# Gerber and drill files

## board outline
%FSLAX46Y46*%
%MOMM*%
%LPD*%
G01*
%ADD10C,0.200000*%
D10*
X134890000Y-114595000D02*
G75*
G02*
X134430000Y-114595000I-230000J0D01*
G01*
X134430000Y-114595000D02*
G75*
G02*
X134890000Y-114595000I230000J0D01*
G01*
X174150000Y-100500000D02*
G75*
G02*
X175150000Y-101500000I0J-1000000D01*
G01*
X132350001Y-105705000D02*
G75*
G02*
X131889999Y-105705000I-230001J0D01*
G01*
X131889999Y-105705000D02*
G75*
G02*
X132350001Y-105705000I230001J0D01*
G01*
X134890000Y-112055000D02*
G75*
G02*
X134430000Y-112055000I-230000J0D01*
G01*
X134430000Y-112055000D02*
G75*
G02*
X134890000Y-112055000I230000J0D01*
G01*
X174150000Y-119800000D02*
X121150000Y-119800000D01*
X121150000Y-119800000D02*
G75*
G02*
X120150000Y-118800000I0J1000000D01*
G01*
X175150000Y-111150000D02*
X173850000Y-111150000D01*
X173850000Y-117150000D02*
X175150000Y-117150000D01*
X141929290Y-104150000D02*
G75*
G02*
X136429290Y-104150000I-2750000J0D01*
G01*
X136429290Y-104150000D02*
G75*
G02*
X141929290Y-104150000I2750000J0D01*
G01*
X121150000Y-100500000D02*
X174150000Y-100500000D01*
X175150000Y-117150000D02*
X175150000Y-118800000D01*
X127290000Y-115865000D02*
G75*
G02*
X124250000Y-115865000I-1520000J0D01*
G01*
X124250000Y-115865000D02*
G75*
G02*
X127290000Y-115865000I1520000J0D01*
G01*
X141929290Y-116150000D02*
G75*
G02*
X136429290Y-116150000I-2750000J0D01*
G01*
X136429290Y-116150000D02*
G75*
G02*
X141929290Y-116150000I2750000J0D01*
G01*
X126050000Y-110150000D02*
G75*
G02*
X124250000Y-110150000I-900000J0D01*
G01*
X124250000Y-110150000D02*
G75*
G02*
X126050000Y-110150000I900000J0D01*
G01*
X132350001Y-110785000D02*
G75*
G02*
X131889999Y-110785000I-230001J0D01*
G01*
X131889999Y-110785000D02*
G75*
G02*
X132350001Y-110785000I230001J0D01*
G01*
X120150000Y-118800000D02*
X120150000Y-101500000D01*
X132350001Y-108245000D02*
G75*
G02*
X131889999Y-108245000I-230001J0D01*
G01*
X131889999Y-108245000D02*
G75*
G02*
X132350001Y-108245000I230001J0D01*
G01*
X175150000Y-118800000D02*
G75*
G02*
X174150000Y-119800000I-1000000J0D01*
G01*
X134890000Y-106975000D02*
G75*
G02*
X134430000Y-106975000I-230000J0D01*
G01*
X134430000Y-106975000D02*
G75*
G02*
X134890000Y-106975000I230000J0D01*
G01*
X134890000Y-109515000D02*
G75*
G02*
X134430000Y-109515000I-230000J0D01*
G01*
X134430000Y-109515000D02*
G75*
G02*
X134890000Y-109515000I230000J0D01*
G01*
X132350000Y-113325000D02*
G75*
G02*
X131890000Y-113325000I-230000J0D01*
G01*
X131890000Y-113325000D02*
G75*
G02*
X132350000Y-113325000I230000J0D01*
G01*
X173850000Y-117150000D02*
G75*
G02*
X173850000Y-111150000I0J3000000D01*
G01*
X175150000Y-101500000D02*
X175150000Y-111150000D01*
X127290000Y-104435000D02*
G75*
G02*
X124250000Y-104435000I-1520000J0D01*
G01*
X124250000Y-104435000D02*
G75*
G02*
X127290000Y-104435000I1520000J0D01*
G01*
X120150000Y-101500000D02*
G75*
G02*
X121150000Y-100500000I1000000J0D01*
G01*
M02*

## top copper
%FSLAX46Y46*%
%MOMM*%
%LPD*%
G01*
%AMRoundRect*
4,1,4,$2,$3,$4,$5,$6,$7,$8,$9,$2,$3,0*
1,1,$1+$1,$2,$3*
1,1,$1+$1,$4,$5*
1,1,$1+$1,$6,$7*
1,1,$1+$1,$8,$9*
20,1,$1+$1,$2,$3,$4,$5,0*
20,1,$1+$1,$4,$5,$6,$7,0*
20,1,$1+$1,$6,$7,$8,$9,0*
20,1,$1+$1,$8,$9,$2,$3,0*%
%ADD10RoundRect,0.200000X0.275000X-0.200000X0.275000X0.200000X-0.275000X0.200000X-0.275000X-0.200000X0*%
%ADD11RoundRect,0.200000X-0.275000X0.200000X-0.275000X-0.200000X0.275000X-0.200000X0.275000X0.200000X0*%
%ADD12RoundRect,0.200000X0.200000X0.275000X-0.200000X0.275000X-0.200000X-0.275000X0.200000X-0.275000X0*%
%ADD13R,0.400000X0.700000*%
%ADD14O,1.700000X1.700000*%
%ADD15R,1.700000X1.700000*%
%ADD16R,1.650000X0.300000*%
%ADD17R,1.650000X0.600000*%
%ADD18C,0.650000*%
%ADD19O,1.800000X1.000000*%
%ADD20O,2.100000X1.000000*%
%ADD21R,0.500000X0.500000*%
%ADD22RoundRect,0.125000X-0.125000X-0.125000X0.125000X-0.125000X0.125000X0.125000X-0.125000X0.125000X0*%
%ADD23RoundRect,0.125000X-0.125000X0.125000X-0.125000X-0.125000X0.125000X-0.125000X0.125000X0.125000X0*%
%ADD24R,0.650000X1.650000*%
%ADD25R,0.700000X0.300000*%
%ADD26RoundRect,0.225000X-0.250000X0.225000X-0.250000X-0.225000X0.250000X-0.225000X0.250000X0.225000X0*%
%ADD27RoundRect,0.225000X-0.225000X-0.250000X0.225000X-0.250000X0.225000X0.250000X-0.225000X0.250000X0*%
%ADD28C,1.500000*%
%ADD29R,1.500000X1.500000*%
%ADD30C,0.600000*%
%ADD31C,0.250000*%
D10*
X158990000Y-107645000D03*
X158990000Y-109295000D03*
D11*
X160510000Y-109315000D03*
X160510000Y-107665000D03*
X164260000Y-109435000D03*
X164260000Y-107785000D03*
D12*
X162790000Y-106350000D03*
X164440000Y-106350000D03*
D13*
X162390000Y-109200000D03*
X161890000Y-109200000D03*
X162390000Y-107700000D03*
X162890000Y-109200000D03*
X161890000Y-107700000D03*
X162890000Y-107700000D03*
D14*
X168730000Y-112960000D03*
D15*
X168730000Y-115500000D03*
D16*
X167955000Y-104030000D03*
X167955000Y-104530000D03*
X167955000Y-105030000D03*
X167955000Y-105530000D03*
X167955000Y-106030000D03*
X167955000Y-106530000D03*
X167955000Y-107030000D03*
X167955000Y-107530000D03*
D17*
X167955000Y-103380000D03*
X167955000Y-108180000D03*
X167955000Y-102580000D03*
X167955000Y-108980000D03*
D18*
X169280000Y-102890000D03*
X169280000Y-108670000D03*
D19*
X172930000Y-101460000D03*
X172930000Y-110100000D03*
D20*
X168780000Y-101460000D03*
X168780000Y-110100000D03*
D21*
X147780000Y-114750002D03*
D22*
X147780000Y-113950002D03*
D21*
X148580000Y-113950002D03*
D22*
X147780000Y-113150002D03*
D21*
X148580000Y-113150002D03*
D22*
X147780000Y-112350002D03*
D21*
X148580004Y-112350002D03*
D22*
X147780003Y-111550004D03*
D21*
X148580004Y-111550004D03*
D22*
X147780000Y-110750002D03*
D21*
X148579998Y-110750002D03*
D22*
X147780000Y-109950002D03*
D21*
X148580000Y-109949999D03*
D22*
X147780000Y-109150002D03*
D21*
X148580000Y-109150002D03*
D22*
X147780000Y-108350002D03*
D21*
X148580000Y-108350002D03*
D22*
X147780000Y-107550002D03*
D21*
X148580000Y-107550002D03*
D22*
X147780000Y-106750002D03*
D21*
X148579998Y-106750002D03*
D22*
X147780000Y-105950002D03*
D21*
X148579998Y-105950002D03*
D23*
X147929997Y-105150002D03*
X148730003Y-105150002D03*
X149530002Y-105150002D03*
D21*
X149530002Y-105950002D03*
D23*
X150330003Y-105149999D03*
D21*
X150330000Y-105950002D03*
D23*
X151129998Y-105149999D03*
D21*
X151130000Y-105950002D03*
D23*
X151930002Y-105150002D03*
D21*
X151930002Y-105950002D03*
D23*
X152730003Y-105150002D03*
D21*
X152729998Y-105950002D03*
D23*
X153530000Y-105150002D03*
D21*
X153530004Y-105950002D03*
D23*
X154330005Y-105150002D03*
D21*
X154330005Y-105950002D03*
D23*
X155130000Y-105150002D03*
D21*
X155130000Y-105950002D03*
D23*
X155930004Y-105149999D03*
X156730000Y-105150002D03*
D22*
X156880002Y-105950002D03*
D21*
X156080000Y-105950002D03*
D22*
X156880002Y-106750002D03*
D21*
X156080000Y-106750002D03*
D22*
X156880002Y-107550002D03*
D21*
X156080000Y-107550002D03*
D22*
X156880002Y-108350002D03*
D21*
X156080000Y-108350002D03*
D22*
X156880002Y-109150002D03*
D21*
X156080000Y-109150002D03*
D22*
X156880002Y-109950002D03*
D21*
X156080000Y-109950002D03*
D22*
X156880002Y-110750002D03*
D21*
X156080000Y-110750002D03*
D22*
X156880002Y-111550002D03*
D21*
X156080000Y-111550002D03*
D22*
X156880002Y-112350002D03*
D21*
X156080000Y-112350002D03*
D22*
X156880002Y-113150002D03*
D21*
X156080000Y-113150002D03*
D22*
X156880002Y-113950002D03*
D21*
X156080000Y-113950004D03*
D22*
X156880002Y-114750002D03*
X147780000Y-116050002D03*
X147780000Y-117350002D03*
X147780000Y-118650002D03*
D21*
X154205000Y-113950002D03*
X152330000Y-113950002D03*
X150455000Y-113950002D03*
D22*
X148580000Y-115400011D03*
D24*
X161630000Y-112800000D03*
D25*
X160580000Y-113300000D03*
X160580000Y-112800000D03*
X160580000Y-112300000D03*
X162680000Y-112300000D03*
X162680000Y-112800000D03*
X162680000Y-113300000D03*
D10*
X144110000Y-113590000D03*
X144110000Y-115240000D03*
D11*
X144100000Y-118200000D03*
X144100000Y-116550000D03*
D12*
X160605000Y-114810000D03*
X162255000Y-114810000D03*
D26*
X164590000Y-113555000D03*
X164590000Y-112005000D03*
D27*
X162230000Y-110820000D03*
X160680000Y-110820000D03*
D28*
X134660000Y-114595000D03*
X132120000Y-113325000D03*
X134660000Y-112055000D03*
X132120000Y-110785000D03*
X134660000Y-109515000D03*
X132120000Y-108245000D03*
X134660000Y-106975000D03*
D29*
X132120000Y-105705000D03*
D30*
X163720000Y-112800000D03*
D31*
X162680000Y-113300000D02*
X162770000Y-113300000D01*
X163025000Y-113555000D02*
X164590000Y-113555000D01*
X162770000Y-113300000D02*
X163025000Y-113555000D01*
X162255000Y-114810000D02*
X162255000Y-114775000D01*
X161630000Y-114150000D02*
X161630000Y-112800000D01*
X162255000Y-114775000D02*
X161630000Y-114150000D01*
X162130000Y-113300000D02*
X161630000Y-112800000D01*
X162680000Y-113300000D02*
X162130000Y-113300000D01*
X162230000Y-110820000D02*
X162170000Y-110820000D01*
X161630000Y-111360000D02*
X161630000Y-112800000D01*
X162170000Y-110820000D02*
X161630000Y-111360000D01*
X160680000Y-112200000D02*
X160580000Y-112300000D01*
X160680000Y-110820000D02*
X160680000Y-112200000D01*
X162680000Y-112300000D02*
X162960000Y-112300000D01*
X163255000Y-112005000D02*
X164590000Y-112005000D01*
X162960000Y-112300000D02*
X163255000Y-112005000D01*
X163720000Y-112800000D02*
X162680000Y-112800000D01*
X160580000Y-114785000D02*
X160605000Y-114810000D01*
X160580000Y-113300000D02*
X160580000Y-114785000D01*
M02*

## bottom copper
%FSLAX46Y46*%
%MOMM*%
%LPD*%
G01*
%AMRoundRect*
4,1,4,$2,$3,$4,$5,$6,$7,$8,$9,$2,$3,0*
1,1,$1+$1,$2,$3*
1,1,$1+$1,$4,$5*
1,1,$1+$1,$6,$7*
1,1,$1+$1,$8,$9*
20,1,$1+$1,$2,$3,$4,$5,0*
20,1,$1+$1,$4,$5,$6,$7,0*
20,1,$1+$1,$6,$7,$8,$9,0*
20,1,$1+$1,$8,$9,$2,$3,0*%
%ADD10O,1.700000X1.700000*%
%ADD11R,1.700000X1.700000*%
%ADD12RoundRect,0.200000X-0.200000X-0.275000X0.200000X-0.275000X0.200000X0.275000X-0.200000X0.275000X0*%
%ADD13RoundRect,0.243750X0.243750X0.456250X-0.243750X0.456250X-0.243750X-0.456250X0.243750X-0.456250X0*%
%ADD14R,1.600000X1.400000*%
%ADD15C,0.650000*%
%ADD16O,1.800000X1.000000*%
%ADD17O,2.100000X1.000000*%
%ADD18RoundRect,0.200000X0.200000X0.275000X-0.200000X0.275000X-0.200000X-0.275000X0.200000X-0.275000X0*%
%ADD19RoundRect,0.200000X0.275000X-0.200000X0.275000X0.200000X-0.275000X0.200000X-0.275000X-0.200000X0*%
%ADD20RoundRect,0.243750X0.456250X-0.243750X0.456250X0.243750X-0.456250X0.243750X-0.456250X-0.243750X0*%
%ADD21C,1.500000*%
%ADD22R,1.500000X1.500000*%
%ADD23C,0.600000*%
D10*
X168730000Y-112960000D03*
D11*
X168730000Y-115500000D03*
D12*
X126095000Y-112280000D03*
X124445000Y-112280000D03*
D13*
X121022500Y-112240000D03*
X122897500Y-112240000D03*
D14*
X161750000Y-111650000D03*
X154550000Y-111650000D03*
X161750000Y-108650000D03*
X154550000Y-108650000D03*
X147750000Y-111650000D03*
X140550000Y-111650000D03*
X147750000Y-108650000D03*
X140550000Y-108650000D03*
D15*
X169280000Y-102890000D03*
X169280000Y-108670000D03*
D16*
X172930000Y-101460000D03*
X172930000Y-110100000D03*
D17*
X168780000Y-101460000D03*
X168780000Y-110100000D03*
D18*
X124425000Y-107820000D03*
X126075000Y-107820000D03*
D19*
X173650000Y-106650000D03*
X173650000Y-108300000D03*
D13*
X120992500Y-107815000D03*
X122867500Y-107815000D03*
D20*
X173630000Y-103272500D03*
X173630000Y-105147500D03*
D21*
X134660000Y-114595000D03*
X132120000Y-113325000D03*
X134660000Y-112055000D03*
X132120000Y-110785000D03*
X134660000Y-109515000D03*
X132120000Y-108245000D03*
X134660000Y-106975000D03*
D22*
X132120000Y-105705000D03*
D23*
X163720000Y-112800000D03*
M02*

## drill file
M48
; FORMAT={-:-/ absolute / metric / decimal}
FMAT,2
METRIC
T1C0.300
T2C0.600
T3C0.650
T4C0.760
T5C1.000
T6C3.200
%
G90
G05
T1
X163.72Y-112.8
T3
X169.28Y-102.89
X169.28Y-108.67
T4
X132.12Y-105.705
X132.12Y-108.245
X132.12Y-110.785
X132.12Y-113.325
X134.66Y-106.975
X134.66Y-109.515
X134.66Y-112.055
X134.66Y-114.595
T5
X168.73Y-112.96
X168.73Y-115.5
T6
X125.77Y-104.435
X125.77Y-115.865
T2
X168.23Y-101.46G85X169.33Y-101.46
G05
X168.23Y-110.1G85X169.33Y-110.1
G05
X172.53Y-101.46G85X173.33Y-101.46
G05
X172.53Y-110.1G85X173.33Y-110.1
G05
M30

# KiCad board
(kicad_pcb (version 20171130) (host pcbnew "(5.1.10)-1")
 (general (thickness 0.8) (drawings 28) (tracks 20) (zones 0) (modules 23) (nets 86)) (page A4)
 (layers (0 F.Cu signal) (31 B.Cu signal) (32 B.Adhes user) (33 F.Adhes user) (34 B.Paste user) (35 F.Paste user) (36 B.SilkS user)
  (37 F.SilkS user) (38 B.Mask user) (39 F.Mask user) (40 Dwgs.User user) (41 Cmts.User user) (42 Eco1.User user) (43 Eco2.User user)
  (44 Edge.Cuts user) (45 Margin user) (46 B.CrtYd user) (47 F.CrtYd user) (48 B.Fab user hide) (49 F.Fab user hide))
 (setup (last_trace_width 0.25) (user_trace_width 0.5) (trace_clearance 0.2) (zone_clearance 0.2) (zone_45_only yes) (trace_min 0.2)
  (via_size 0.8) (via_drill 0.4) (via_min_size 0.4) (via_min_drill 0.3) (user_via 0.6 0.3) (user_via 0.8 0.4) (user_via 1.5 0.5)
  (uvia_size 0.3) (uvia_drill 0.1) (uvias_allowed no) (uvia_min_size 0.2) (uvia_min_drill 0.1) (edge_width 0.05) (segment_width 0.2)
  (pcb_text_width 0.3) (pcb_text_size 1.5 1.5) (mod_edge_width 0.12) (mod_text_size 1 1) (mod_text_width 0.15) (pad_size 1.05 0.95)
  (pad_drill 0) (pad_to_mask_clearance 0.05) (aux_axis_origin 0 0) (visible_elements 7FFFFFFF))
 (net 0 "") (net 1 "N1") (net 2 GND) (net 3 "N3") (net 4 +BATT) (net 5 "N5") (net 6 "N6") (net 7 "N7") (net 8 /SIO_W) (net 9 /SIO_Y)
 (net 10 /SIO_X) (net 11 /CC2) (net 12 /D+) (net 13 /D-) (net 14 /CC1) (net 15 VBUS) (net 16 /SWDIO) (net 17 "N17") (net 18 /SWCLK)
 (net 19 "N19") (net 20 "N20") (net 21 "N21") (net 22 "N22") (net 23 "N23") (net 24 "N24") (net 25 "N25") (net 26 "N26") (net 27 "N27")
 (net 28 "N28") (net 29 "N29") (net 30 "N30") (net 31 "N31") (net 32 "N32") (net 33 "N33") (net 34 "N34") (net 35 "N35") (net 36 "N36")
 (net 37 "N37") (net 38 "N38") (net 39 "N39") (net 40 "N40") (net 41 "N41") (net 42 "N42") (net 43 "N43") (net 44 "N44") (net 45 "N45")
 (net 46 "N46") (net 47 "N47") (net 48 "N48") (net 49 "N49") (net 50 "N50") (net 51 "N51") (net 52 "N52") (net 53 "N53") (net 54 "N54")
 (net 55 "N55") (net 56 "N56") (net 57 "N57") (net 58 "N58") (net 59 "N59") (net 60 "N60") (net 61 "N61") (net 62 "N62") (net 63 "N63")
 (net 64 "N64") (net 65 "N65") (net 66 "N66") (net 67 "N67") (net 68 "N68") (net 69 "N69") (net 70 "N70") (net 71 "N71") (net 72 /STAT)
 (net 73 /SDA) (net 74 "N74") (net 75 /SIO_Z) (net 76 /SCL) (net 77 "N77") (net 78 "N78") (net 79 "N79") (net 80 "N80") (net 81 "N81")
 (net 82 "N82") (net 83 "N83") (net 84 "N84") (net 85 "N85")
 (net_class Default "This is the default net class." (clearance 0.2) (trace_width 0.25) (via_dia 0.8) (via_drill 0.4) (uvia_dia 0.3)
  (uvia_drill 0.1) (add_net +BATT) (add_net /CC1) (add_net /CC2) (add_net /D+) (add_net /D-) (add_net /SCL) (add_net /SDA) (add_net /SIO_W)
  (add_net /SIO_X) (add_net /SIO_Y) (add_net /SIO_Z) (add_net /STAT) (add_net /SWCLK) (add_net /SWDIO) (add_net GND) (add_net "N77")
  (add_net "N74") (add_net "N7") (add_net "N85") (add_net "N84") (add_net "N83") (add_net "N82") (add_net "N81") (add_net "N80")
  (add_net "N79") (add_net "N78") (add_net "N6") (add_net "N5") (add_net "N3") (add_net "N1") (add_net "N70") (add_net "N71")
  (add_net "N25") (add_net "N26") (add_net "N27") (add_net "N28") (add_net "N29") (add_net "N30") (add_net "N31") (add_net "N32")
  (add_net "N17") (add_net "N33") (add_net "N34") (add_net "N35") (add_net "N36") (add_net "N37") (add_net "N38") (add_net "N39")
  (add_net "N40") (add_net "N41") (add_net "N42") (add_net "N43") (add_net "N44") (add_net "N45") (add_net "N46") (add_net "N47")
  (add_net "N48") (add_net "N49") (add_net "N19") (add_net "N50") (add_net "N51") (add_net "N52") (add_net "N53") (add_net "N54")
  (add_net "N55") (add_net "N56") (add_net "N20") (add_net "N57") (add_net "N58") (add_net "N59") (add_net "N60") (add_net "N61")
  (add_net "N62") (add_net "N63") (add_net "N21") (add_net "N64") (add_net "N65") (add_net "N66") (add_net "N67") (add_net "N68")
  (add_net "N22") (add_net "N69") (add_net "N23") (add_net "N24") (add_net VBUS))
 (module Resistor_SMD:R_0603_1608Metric (layer F.Cu) (at 158.99 108.47 90)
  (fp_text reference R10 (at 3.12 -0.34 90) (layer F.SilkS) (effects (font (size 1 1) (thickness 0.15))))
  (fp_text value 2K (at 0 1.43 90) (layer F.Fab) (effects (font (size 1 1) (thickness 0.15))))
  (pad 2 smd roundrect (at 0.825 0 90) (size 0.8 0.95) (layers F.Cu F.Paste F.Mask) (roundrect_rratio 0.25) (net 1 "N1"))
  (pad 1 smd roundrect (at -0.825 0 90) (size 0.8 0.95) (layers F.Cu F.Paste F.Mask) (roundrect_rratio 0.25) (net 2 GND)))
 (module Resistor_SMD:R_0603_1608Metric (layer F.Cu) (at 160.51 108.49 270)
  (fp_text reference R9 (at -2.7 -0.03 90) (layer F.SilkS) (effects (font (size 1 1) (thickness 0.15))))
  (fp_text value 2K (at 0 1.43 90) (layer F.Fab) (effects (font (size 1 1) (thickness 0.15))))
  (pad 2 smd roundrect (at 0.825 0 270) (size 0.8 0.95) (layers F.Cu F.Paste F.Mask) (roundrect_rratio 0.25) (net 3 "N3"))
  (pad 1 smd roundrect (at -0.825 0 270) (size 0.8 0.95) (layers F.Cu F.Paste F.Mask) (roundrect_rratio 0.25) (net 1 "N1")))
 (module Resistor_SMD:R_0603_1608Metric (layer F.Cu) (at 164.26 108.61 270)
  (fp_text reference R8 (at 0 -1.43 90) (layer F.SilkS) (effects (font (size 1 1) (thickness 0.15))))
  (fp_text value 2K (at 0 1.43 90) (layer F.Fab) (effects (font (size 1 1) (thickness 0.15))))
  (pad 2 smd roundrect (at 0.825 0 270) (size 0.8 0.95) (layers F.Cu F.Paste F.Mask) (roundrect_rratio 0.25) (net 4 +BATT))
  (pad 1 smd roundrect (at -0.825 0 270) (size 0.8 0.95) (layers F.Cu F.Paste F.Mask) (roundrect_rratio 0.25) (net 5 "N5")))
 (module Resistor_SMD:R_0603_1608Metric (layer F.Cu) (at 163.615 106.35 180)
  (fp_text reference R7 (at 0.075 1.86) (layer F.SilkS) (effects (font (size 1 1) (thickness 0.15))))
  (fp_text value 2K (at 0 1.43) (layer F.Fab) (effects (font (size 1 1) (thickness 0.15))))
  (pad 2 smd roundrect (at 0.825 0 180) (size 0.8 0.95) (layers F.Cu F.Paste F.Mask) (roundrect_rratio 0.25) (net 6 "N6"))
  (pad 1 smd roundrect (at -0.825 0 180) (size 0.8 0.95) (layers F.Cu F.Paste F.Mask) (roundrect_rratio 0.25) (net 2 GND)))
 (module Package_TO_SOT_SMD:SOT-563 (layer F.Cu) (at 162.39 108.45 270)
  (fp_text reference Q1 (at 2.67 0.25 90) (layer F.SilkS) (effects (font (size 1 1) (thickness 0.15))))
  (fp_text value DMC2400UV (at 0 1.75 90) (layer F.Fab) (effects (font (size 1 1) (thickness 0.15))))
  (pad 5 smd rect (at 0.75 0 270) (size 0.7 0.4) (layers F.Cu F.Paste F.Mask) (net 5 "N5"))
  (pad 4 smd rect (at 0.75 0.5 270) (size 0.7 0.4) (layers F.Cu F.Paste F.Mask) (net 3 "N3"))
  (pad 2 smd rect (at -0.75 0 270) (size 0.7 0.4) (layers F.Cu F.Paste F.Mask) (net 6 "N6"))
  (pad 6 smd rect (at 0.75 -0.5 270) (size 0.7 0.4) (layers F.Cu F.Paste F.Mask) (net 4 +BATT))
  (pad 3 smd rect (at -0.75 0.5 270) (size 0.7 0.4) (layers F.Cu F.Paste F.Mask) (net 5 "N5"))
  (pad 1 smd rect (at -0.75 -0.5 270) (size 0.7 0.4) (layers F.Cu F.Paste F.Mask) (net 2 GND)))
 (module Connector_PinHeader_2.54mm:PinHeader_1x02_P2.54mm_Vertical (layer F.Cu) (at 168.73 115.5 180)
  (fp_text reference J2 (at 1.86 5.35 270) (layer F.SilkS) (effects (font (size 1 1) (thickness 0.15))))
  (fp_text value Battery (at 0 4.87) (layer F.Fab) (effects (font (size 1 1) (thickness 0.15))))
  (pad 2 thru_hole oval (at 0 2.54 180) (size 1.7 1.7) (drill 1) (layers *.Cu *.Mask) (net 4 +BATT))
  (pad 1 thru_hole rect (at 0 0 180) (size 1.7 1.7) (drill 1) (layers *.Cu *.Mask) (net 2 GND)))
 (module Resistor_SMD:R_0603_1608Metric (layer B.Cu) (at 125.27 112.28)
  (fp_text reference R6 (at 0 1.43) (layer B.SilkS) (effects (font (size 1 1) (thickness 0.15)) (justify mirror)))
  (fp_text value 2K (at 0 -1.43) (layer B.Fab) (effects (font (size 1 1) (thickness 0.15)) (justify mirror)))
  (pad 2 smd roundrect (at 0.825 0) (size 0.8 0.95) (layers B.Cu B.Paste B.Mask) (roundrect_rratio 0.25) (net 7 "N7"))
  (pad 1 smd roundrect (at -0.825 0) (size 0.8 0.95) (layers B.Cu B.Paste B.Mask) (roundrect_rratio 0.25) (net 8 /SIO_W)))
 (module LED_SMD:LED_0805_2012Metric (layer B.Cu) (at 121.96 112.24 180)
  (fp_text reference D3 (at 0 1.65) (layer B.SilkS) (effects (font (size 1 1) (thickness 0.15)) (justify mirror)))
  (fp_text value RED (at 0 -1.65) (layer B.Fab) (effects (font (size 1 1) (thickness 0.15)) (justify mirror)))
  (pad 2 smd roundrect (at 0.9375 0 180) (size 0.975 1.4) (layers B.Cu B.Paste B.Mask) (roundrect_rratio 0.25) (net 4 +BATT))
  (pad 1 smd roundrect (at -0.9375 0 180) (size 0.975 1.4) (layers B.Cu B.Paste B.Mask) (roundrect_rratio 0.25) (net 7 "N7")))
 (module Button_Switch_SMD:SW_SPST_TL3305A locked (layer B.Cu) (at 158.15 110.15 180)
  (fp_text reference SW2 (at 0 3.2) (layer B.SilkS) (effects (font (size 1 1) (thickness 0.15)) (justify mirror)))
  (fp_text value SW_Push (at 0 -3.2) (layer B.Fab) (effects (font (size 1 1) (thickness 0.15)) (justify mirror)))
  (pad 2 smd rect (at -3.6 -1.5 180) (size 1.6 1.4) (layers B.Cu B.Paste B.Mask) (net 2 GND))
  (pad 2 smd rect (at 3.6 -1.5 180) (size 1.6 1.4) (layers B.Cu B.Paste B.Mask) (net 2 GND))
  (pad 1 smd rect (at -3.6 1.5 180) (size 1.6 1.4) (layers B.Cu B.Paste B.Mask) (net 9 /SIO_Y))
  (pad 1 smd rect (at 3.6 1.5 180) (size 1.6 1.4) (layers B.Cu B.Paste B.Mask) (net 9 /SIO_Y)))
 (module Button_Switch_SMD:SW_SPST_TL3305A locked (layer B.Cu) (at 144.15 110.15 180)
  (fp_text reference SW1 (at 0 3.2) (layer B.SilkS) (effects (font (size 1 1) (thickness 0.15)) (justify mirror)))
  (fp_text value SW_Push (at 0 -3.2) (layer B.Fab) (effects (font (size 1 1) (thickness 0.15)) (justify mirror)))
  (pad 2 smd rect (at -3.6 -1.5 180) (size 1.6 1.4) (layers B.Cu B.Paste B.Mask) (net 2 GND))
  (pad 2 smd rect (at 3.6 -1.5 180) (size 1.6 1.4) (layers B.Cu B.Paste B.Mask) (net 2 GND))
  (pad 1 smd rect (at -3.6 1.5 180) (size 1.6 1.4) (layers B.Cu B.Paste B.Mask) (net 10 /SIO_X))
  (pad 1 smd rect (at 3.6 1.5 180) (size 1.6 1.4) (layers B.Cu B.Paste B.Mask) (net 10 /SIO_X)))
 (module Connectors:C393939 (layer F.Cu) (at 168.78 105.78 90)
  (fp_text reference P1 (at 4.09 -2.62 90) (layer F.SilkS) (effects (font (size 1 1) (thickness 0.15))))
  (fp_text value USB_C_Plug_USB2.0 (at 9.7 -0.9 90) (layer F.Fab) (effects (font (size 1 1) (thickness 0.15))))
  (pad B5 smd rect (at 1.75 -0.825 90) (size 0.3 1.65) (layers F.Cu F.Paste F.Mask) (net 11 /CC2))
  (pad B8 smd rect (at 1.25 -0.825 90) (size 0.3 1.65) (layers F.Cu F.Paste F.Mask))
  (pad A6 smd rect (at 0.75 -0.825 90) (size 0.3 1.65) (layers F.Cu F.Paste F.Mask) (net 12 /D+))
  (pad A7 smd rect (at 0.25 -0.825 90) (size 0.3 1.65) (layers F.Cu F.Paste F.Mask) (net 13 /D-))
  (pad A6 smd rect (at -0.25 -0.825 90) (size 0.3 1.65) (layers F.Cu F.Paste F.Mask) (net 12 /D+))
  (pad A7 smd rect (at -0.75 -0.825 90) (size 0.3 1.65) (layers F.Cu F.Paste F.Mask) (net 13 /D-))
  (pad A5 smd rect (at -1.25 -0.825 90) (size 0.3 1.65) (layers F.Cu F.Paste F.Mask) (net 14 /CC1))
  (pad A8 smd rect (at -1.75 -0.825 90) (size 0.3 1.65) (layers F.Cu F.Paste F.Mask))
  (pad A4 smd rect (at 2.4 -0.825 90) (size 0.6 1.65) (layers F.Cu F.Paste F.Mask) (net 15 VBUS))
  (pad A4 smd rect (at -2.4 -0.825 90) (size 0.6 1.65) (layers F.Cu F.Paste F.Mask) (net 15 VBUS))
  (pad A1 smd rect (at 3.2 -0.825 90) (size 0.6 1.65) (layers F.Cu F.Paste F.Mask) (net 2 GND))
  (pad A1 smd rect (at -3.2 -0.825 90) (size 0.6 1.65) (layers F.Cu F.Paste F.Mask) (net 2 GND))
  (pad "" thru_hole circle (at 2.89 0.5 90) (size 0.65 0.65) (drill 0.65) (layers *.Cu *.Mask))
  (pad "" thru_hole circle (at -2.89 0.5 90) (size 0.65 0.65) (drill 0.65) (layers *.Cu *.Mask))
  (pad S1 thru_hole oval (at 4.32 4.15 90) (size 1 1.8) (drill oval 0.6 1.4) (layers *.Cu *.Mask) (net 2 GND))
  (pad S1 thru_hole oval (at -4.32 4.15 90) (size 1 1.8) (drill oval 0.6 1.4) (layers *.Cu *.Mask) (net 2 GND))
  (pad S1 thru_hole oval (at 4.32 0 90) (size 1 2.1) (drill oval 0.6 1.7) (layers *.Cu *.Mask) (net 2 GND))
  (pad S1 thru_hole oval (at -4.32 0 90) (size 1 2.1) (drill oval 0.6 1.7) (layers *.Cu *.Mask) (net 2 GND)))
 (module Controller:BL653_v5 (layer F.Cu) (at 152.33 111.9 270)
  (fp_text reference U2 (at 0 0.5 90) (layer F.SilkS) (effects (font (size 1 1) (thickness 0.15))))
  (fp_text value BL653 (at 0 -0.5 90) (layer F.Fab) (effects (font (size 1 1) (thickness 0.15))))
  (pad 0 smd rect (at 2.850002 4.55) (size 0.5 0.5) (layers F.Cu F.Paste F.Mask) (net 2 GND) (solder_mask_margin 0.0508))
  (pad 1 smd roundrect (at 2.050002 4.55) (size 0.5 0.5) (layers F.Cu F.Paste F.Mask) (roundrect_rratio 0.25) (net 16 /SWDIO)
   (solder_mask_margin 0.0508))
  (pad 2 smd rect (at 2.050002 3.75 270) (size 0.5 0.5) (layers F.Cu F.Paste F.Mask) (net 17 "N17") (solder_mask_margin 0.0508))
  (pad 3 smd roundrect (at 1.250002 4.55) (size 0.5 0.5) (layers F.Cu F.Paste F.Mask) (roundrect_rratio 0.25) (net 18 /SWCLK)
   (solder_mask_margin 0.0508))
  (pad 4 smd rect (at 1.250002 3.75 270) (size 0.5 0.5) (layers F.Cu F.Paste F.Mask) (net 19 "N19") (solder_mask_margin 0.0508))
  (pad 5 smd roundrect (at 0.450002 4.55) (size 0.5 0.5) (layers F.Cu F.Paste F.Mask) (roundrect_rratio 0.25) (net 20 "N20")
   (solder_mask_margin 0.0508))
  (pad 6 smd rect (at 0.450002 3.749996 270) (size 0.5 0.5) (layers F.Cu F.Paste F.Mask) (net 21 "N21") (solder_mask_margin 0.0508))
  (pad 7 smd roundrect (at -0.349996 4.549997) (size 0.5 0.5) (layers F.Cu F.Paste F.Mask) (roundrect_rratio 0.25) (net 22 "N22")
   (solder_mask_margin 0.0508))
  (pad 8 smd rect (at -0.349996 3.749996 270) (size 0.5 0.5) (layers F.Cu F.Paste F.Mask) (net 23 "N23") (solder_mask_margin 0.0508))
  (pad 9 smd roundrect (at -1.149998 4.55) (size 0.5 0.5) (layers F.Cu F.Paste F.Mask) (roundrect_rratio 0.25) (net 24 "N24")
   (solder_mask_margin 0.0508))
  (pad 10 smd rect (at -1.149998 3.750002 270) (size 0.5 0.5) (layers F.Cu F.Paste F.Mask) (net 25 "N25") (solder_mask_margin 0.0508))
  (pad 11 smd roundrect (at -1.949998 4.55) (size 0.5 0.5) (layers F.Cu F.Paste F.Mask) (roundrect_rratio 0.25) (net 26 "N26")
   (solder_mask_margin 0.0508))
  (pad 12 smd rect (at -1.950001 3.75 270) (size 0.5 0.5) (layers F.Cu F.Paste F.Mask) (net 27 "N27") (solder_mask_margin 0.0508))
  (pad 13 smd roundrect (at -2.749998 4.55) (size 0.5 0.5) (layers F.Cu F.Paste F.Mask) (roundrect_rratio 0.25) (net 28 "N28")
   (solder_mask_margin 0.0508))
  (pad 14 smd rect (at -2.749998 3.75 270) (size 0.5 0.5) (layers F.Cu F.Paste F.Mask) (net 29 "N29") (solder_mask_margin 0.0508))
  (pad 15 smd roundrect (at -3.549998 4.55) (size 0.5 0.5) (layers F.Cu F.Paste F.Mask) (roundrect_rratio 0.25) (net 12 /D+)
   (solder_mask_margin 0.0508))
  (pad 16 smd rect (at -3.549998 3.75 270) (size 0.5 0.5) (layers F.Cu F.Paste F.Mask) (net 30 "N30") (solder_mask_margin 0.0508))
  (pad 17 smd roundrect (at -4.349998 4.55) (size 0.5 0.5) (layers F.Cu F.Paste F.Mask) (roundrect_rratio 0.25) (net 13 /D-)
   (solder_mask_margin 0.0508))
  (pad 18 smd rect (at -4.349998 3.75 270) (size 0.5 0.5) (layers F.Cu F.Paste F.Mask) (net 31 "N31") (solder_mask_margin 0.0508))
  (pad 19 smd roundrect (at -5.149998 4.55) (size 0.5 0.5) (layers F.Cu F.Paste F.Mask) (roundrect_rratio 0.25) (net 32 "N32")
   (solder_mask_margin 0.0508))
  (pad 20 smd rect (at -5.149998 3.750002 270) (size 0.5 0.5) (layers F.Cu F.Paste F.Mask) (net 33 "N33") (solder_mask_margin 0.0508))
  (pad 21 smd roundrect (at -5.949998 4.55) (size 0.5 0.5) (layers F.Cu F.Paste F.Mask) (roundrect_rratio 0.25) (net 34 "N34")
   (solder_mask_margin 0.0508))
  (pad 22 smd rect (at -5.949998 3.750002 270) (size 0.5 0.5) (layers F.Cu F.Paste F.Mask) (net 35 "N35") (solder_mask_margin 0.0508))
  (pad 23 smd roundrect (at -6.749998 4.400003 270) (size 0.5 0.5) (layers F.Cu F.Paste F.Mask) (roundrect_rratio 0.25) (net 2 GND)
   (solder_mask_margin 0.0508))
  (pad 24 smd roundrect (at -6.749998 3.599997 270) (size 0.5 0.5) (layers F.Cu F.Paste F.Mask) (roundrect_rratio 0.25) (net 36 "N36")
   (solder_mask_margin 0.0508))
  (pad 25 smd roundrect (at -6.749998 2.799998 270) (size 0.5 0.5) (layers F.Cu F.Paste F.Mask) (roundrect_rratio 0.25) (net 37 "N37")
   (solder_mask_margin 0.0508))
  (pad 26 smd rect (at -5.949998 2.799998 270) (size 0.5 0.5) (layers F.Cu F.Paste F.Mask) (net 2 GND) (solder_mask_margin 0.0508))
  (pad 27 smd roundrect (at -6.750001 1.999997 270) (size 0.5 0.5) (layers F.Cu F.Paste F.Mask) (roundrect_rratio 0.25) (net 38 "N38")
   (solder_mask_margin 0.0508))
  (pad 28 smd rect (at -5.949998 2 270) (size 0.5 0.5) (layers F.Cu F.Paste F.Mask) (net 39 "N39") (solder_mask_margin 0.0508))
  (pad 29 smd roundrect (at -6.750001 1.200002 270) (size 0.5 0.5) (layers F.Cu F.Paste F.Mask) (roundrect_rratio 0.25) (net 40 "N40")
   (solder_mask_margin 0.0508))
  (pad 30 smd rect (at -5.949998 1.2 270) (size 0.5 0.5) (layers F.Cu F.Paste F.Mask) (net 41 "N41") (solder_mask_margin 0.0508))
  (pad 31 smd roundrect (at -6.749998 0.399998 270) (size 0.5 0.5) (layers F.Cu F.Paste F.Mask) (roundrect_rratio 0.25) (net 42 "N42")
   (solder_mask_margin 0.0508))
  (pad 32 smd rect (at -5.949998 0.399998 270) (size 0.5 0.5) (layers F.Cu F.Paste F.Mask) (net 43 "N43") (solder_mask_margin 0.0508))
  (pad 33 smd roundrect (at -6.749998 -0.400003 270) (size 0.5 0.5) (layers F.Cu F.Paste F.Mask) (roundrect_rratio 0.25) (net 2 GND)
   (solder_mask_margin 0.0508))
  (pad 34 smd rect (at -5.949998 -0.399998 270) (size 0.5 0.5) (layers F.Cu F.Paste F.Mask) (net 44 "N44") (solder_mask_margin 0.0508))
  (pad 35 smd roundrect (at -6.749998 -1.2 270) (size 0.5 0.5) (layers F.Cu F.Paste F.Mask) (roundrect_rratio 0.25) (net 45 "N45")
   (solder_mask_margin 0.0508))
  (pad 36 smd rect (at -5.949998 -1.200004 270) (size 0.5 0.5) (layers F.Cu F.Paste F.Mask) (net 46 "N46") (solder_mask_margin 0.0508))
  (pad 37 smd roundrect (at -6.749998 -2.000005 270) (size 0.5 0.5) (layers F.Cu F.Paste F.Mask) (roundrect_rratio 0.25) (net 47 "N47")
   (solder_mask_margin 0.0508))
  (pad 38 smd rect (at -5.949998 -2.000005 270) (size 0.5 0.5) (layers F.Cu F.Paste F.Mask) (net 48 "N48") (solder_mask_margin 0.0508))
  (pad 39 smd roundrect (at -6.749998 -2.8 270) (size 0.5 0.5) (layers F.Cu F.Paste F.Mask) (roundrect_rratio 0.25) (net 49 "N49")
   (solder_mask_margin 0.0508))
  (pad 40 smd rect (at -5.949998 -2.8 270) (size 0.5 0.5) (layers F.Cu F.Paste F.Mask) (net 2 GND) (solder_mask_margin 0.0508))
  (pad 41 smd roundrect (at -6.750001 -3.600004 270) (size 0.5 0.5) (layers F.Cu F.Paste F.Mask) (roundrect_rratio 0.25) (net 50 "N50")
   (solder_mask_margin 0.0508))
  (pad 42 smd roundrect (at -6.749998 -4.4 270) (size 0.5 0.5) (layers F.Cu F.Paste F.Mask) (roundrect_rratio 0.25) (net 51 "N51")
   (solder_mask_margin 0.0508))
  (pad 43 smd roundrect (at -5.949998 -4.550002) (size 0.5 0.5) (layers F.Cu F.Paste F.Mask) (roundrect_rratio 0.25) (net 2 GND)
   (solder_mask_margin 0.0508))
  (pad 44 smd rect (at -5.949998 -3.75 270) (size 0.5 0.5) (layers F.Cu F.Paste F.Mask) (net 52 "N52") (solder_mask_margin 0.0508))
  (pad 45 smd roundrect (at -5.149998 -4.550002) (size 0.5 0.5) (layers F.Cu F.Paste F.Mask) (roundrect_rratio 0.25) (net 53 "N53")
   (solder_mask_margin 0.0508))
  (pad 46 smd rect (at -5.149998 -3.75 270) (size 0.5 0.5) (layers F.Cu F.Paste F.Mask) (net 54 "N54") (solder_mask_margin 0.0508))
  (pad 47 smd roundrect (at -4.349998 -4.550002) (size 0.5 0.5) (layers F.Cu F.Paste F.Mask) (roundrect_rratio 0.25) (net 2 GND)
   (solder_mask_margin 0.0508))
  (pad 48 smd rect (at -4.349998 -3.75 270) (size 0.5 0.5) (layers F.Cu F.Paste F.Mask) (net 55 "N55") (solder_mask_margin 0.0508))
  (pad 49 smd roundrect (at -3.549998 -4.550002) (size 0.5 0.5) (layers F.Cu F.Paste F.Mask) (roundrect_rratio 0.25) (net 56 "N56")
   (solder_mask_margin 0.0508))
  (pad 50 smd rect (at -3.549998 -3.75 270) (size 0.5 0.5) (layers F.Cu F.Paste F.Mask) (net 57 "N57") (solder_mask_margin 0.0508))
  (pad 51 smd roundrect (at -2.749998 -4.550002) (size 0.5 0.5) (layers F.Cu F.Paste F.Mask) (roundrect_rratio 0.25) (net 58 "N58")
   (solder_mask_margin 0.0508))
  (pad 52 smd rect (at -2.749998 -3.75 270) (size 0.5 0.5) (layers F.Cu F.Paste F.Mask) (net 2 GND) (solder_mask_margin 0.0508))
  (pad 53 smd roundrect (at -1.949998 -4.550002) (size 0.5 0.5) (layers F.Cu F.Paste F.Mask) (roundrect_rratio 0.25) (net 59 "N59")
   (solder_mask_margin 0.0508))
  (pad 54 smd rect (at -1.949998 -3.75 270) (size 0.5 0.5) (layers F.Cu F.Paste F.Mask) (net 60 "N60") (solder_mask_margin 0.0508))
  (pad 55 smd roundrect (at -1.149998 -4.550002) (size 0.5 0.5) (layers F.Cu F.Paste F.Mask) (roundrect_rratio 0.25) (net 2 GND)
   (solder_mask_margin 0.0508))
  (pad 56 smd rect (at -1.149998 -3.75 270) (size 0.5 0.5) (layers F.Cu F.Paste F.Mask) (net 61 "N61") (solder_mask_margin 0.0508))
  (pad 57 smd roundrect (at -0.349998 -4.550002) (size 0.5 0.5) (layers F.Cu F.Paste F.Mask) (roundrect_rratio 0.25) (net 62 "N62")
   (solder_mask_margin 0.0508))
  (pad 58 smd rect (at -0.349998 -3.75 270) (size 0.5 0.5) (layers F.Cu F.Paste F.Mask) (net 2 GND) (solder_mask_margin 0.0508))
  (pad 59 smd roundrect (at 0.450002 -4.550002) (size 0.5 0.5) (layers F.Cu F.Paste F.Mask) (roundrect_rratio 0.25) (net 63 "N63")
   (solder_mask_margin 0.0508))
  (pad 60 smd rect (at 0.450002 -3.75 270) (size 0.5 0.5) (layers F.Cu F.Paste F.Mask) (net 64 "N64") (solder_mask_margin 0.0508))
  (pad 61 smd roundrect (at 1.250002 -4.550002) (size 0.5 0.5) (layers F.Cu F.Paste F.Mask) (roundrect_rratio 0.25) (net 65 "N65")
   (solder_mask_margin 0.0508))
  (pad 62 smd rect (at 1.250002 -3.75 270) (size 0.5 0.5) (layers F.Cu F.Paste F.Mask) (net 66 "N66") (solder_mask_margin 0.0508))
  (pad 63 smd roundrect (at 2.050002 -4.550002) (size 0.5 0.5) (layers F.Cu F.Paste F.Mask) (roundrect_rratio 0.25) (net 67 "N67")
   (solder_mask_margin 0.0508))
  (pad 64 smd rect (at 2.050004 -3.75 270) (size 0.5 0.5) (layers F.Cu F.Paste F.Mask) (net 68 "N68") (solder_mask_margin 0.0508))
  (pad 65 smd roundrect (at 2.850002 -4.550002) (size 0.5 0.5) (layers F.Cu F.Paste F.Mask) (roundrect_rratio 0.25) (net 2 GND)
   (solder_mask_margin 0.0508))
  (pad 66 smd roundrect (at 4.150002 4.55) (size 0.5 0.5) (layers F.Cu F.Paste F.Mask) (roundrect_rratio 0.25) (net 2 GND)
   (solder_mask_margin 0.0508))
  (pad 67 smd roundrect (at 5.450002 4.55) (size 0.5 0.5) (layers F.Cu F.Paste F.Mask) (roundrect_rratio 0.25) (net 2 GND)
   (solder_mask_margin 0.0508))
  (pad 68 smd roundrect (at 6.750002 4.55) (size 0.5 0.5) (layers F.Cu F.Paste F.Mask) (roundrect_rratio 0.25) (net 2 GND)
   (solder_mask_margin 0.0508))
  (pad 69 smd rect (at 2.050002 -1.875 270) (size 0.5 0.5) (layers F.Cu F.Paste F.Mask) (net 2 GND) (solder_mask_margin 0.0508))
  (pad 70 smd rect (at 2.050002 0 270) (size 0.5 0.5) (layers F.Cu F.Paste F.Mask) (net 2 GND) (solder_mask_margin 0.0508))
  (pad 71 smd rect (at 2.050002 1.875 270) (size 0.5 0.5) (layers F.Cu F.Paste F.Mask) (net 2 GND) (solder_mask_margin 0.0508))
  (pad 72 smd roundrect (at 3.500011 3.75) (size 0.5 0.5) (layers F.Cu F.Paste F.Mask) (roundrect_rratio 0.25) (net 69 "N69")
   (solder_mask_margin 0.0508)))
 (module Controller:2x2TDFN (layer F.Cu) (at 161.63 112.8 180)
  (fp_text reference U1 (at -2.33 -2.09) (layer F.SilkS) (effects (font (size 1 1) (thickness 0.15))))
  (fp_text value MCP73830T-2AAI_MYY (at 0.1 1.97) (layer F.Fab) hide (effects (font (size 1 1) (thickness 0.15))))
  (pad 7 smd rect (at 0 0 180) (size 0.65 1.65) (layers F.Cu F.Paste F.Mask) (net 2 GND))
  (pad 6 smd rect (at 1.05 -0.5 270) (size 0.3 0.7) (layers F.Cu F.Paste F.Mask) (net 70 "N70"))
  (pad 5 smd rect (at 1.05 0 270) (size 0.3 0.7) (layers F.Cu F.Paste F.Mask) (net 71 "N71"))
  (pad 4 smd rect (at 1.05 0.5 270) (size 0.3 0.7) (layers F.Cu F.Paste F.Mask) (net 15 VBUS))
  (pad 3 smd rect (at -1.05 0.5 270) (size 0.3 0.7) (layers F.Cu F.Paste F.Mask) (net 4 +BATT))
  (pad 2 smd rect (at -1.05 0 270) (size 0.3 0.7) (layers F.Cu F.Paste F.Mask) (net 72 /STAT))
  (pad 1 smd rect (at -1.05 -0.5 270) (size 0.3 0.7) (layers F.Cu F.Paste F.Mask) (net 2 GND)))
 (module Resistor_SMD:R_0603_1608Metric (layer F.Cu) (at 144.11 114.415 90)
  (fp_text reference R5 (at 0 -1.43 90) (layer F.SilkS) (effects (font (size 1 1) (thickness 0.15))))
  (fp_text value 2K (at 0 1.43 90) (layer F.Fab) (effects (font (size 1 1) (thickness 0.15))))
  (pad 2 smd roundrect (at 0.825 0 90) (size 0.8 0.95) (layers F.Cu F.Paste F.Mask) (roundrect_rratio 0.25) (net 4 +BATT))
  (pad 1 smd roundrect (at -0.825 0 90) (size 0.8 0.95) (layers F.Cu F.Paste F.Mask) (roundrect_rratio 0.25) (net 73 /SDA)))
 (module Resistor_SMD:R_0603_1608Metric (layer B.Cu) (at 125.25 107.82 180)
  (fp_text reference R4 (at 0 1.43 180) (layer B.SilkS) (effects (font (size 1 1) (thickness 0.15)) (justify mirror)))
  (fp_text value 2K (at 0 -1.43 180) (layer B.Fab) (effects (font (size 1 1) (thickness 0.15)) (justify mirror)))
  (pad 2 smd roundrect (at 0.825 0 180) (size 0.8 0.95) (layers B.Cu B.Paste B.Mask) (roundrect_rratio 0.25) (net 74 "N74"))
  (pad 1 smd roundrect (at -0.825 0 180) (size 0.8 0.95) (layers B.Cu B.Paste B.Mask) (roundrect_rratio 0.25) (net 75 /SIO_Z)))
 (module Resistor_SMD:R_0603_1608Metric (layer F.Cu) (at 144.1 117.375 270)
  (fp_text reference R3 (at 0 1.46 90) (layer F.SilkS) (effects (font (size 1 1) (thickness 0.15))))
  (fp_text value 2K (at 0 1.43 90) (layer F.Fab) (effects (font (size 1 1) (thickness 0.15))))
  (pad 2 smd roundrect (at 0.825 0 270) (size 0.8 0.95) (layers F.Cu F.Paste F.Mask) (roundrect_rratio 0.25) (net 4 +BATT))
  (pad 1 smd roundrect (at -0.825 0 270) (size 0.8 0.95) (layers F.Cu F.Paste F.Mask) (roundrect_rratio 0.25) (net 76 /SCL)))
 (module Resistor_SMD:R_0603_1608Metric (layer F.Cu) (at 161.43 114.81 180)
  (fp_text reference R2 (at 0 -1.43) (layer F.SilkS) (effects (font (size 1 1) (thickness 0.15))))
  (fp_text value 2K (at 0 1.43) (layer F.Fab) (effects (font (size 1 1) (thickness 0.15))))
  (pad 2 smd roundrect (at 0.825 0 180) (size 0.8 0.95) (layers F.Cu F.Paste F.Mask) (roundrect_rratio 0.25) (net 70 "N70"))
  (pad 1 smd roundrect (at -0.825 0 180) (size 0.8 0.95) (layers F.Cu F.Paste F.Mask) (roundrect_rratio 0.25) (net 2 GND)))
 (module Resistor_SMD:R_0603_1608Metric (layer B.Cu) (at 173.65 107.475 90)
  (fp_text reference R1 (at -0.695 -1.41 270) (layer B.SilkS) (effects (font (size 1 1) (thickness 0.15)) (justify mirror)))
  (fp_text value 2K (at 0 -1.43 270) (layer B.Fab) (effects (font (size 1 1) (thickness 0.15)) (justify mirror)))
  (pad 2 smd roundrect (at 0.825 0 90) (size 0.8 0.95) (layers B.Cu B.Paste B.Mask) (roundrect_rratio 0.25) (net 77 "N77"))
  (pad 1 smd roundrect (at -0.825 0 90) (size 0.8 0.95) (layers B.Cu B.Paste B.Mask) (roundrect_rratio 0.25) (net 72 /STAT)))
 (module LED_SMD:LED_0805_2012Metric (layer B.Cu) (at 121.93 107.815 180)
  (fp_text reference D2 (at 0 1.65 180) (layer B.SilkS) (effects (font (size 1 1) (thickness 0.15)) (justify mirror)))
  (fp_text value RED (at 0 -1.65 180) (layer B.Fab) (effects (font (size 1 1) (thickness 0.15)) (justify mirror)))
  (pad 2 smd roundrect (at 0.9375 0 180) (size 0.975 1.4) (layers B.Cu B.Paste B.Mask) (roundrect_rratio 0.25) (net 4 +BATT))
  (pad 1 smd roundrect (at -0.9375 0 180) (size 0.975 1.4) (layers B.Cu B.Paste B.Mask) (roundrect_rratio 0.25) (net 74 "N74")))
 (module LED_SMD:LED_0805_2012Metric (layer B.Cu) (at 173.63 104.21 90)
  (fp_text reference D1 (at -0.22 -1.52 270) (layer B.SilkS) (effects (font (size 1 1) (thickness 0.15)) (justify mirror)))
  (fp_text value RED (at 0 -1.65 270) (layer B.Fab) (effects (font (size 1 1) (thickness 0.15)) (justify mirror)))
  (pad 2 smd roundrect (at 0.9375 0 90) (size 0.975 1.4) (layers B.Cu B.Paste B.Mask) (roundrect_rratio 0.25) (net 15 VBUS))
  (pad 1 smd roundrect (at -0.9375 0 90) (size 0.975 1.4) (layers B.Cu B.Paste B.Mask) (roundrect_rratio 0.25) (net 77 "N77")))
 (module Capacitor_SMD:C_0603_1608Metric (layer F.Cu) (at 164.59 112.78 270)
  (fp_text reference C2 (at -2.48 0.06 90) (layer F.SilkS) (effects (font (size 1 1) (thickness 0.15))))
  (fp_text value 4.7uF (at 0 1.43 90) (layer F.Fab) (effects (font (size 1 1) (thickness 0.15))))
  (pad 2 smd roundrect (at 0.775 0 270) (size 0.9 0.95) (layers F.Cu F.Paste F.Mask) (roundrect_rratio 0.25) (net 2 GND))
  (pad 1 smd roundrect (at -0.775 0 270) (size 0.9 0.95) (layers F.Cu F.Paste F.Mask) (roundrect_rratio 0.25) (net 4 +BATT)))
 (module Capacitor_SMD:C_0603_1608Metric (layer F.Cu) (at 161.455 110.82)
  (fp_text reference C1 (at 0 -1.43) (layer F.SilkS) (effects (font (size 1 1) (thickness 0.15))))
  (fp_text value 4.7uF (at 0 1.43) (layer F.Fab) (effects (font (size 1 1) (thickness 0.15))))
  (pad 2 smd roundrect (at 0.775 0) (size 0.9 0.95) (layers F.Cu F.Paste F.Mask) (roundrect_rratio 0.25) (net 2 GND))
  (pad 1 smd roundrect (at -0.775 0) (size 0.9 0.95) (layers F.Cu F.Paste F.Mask) (roundrect_rratio 0.25) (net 15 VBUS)))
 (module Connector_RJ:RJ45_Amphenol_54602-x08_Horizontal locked (layer F.Cu) (at 132.12 105.705 270)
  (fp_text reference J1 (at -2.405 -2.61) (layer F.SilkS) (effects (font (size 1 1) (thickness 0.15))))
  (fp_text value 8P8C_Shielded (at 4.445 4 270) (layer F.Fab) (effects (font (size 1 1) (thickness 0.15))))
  (pad 8 thru_hole circle (at 8.89 -2.54 270) (size 1.5 1.5) (drill 0.76) (layers *.Cu *.Mask) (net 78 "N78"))
  (pad 7 thru_hole circle (at 7.62 0 270) (size 1.5 1.5) (drill 0.76) (layers *.Cu *.Mask) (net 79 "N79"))
  (pad 6 thru_hole circle (at 6.35 -2.54 270) (size 1.5 1.5) (drill 0.76) (layers *.Cu *.Mask) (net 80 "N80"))
  (pad 5 thru_hole circle (at 5.08 0 270) (size 1.5 1.5) (drill 0.76) (layers *.Cu *.Mask) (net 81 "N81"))
  (pad 4 thru_hole circle (at 3.81 -2.54 270) (size 1.5 1.5) (drill 0.76) (layers *.Cu *.Mask) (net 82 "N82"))
  (pad 3 thru_hole circle (at 2.54 0 270) (size 1.5 1.5) (drill 0.76) (layers *.Cu *.Mask) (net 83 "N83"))
  (pad 2 thru_hole circle (at 1.27 -2.54 270) (size 1.5 1.5) (drill 0.76) (layers *.Cu *.Mask) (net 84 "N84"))
  (pad 1 thru_hole rect (at 0 0 270) (size 1.5 1.5) (drill 0.76) (layers *.Cu *.Mask) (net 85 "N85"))
  (pad "" np_thru_hole circle (at -1.27 6.35 270) (size 3.2 3.2) (drill 3.2) (layers *.Cu *.Mask))
  (pad "" np_thru_hole circle (at 10.16 6.35 270) (size 3.2 3.2) (drill 3.2) (layers *.Cu *.Mask)))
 (gr_circle (center 134.66 114.595) (end 134.89 114.595) (layer Edge.Cuts) (width 0.2))
 (gr_arc (start 174.15 101.5) (end 175.15 101.5) (angle -90) (layer Edge.Cuts) (width 0.2))
 (gr_circle (center 132.12 105.705) (end 132.350001 105.705) (layer Edge.Cuts) (width 0.2))
 (gr_circle (center 134.66 112.055) (end 134.89 112.055) (layer Edge.Cuts) (width 0.2))
 (gr_line (start 174.15 119.8) (end 121.15 119.8) (layer Edge.Cuts) (width 0.2))
 (gr_arc (start 121.15 118.8) (end 120.15 118.8) (angle -90) (layer Edge.Cuts) (width 0.2))
 (gr_line (start 175.15 111.15) (end 173.85 111.15) (layer Edge.Cuts) (width 0.2))
 (gr_line (start 173.85 117.15) (end 175.15 117.15) (layer Edge.Cuts) (width 0.2))
 (gr_circle (center 139.17929 104.15) (end 141.92929 104.15) (layer Edge.Cuts) (width 0.2))
 (gr_line (start 121.15 100.5) (end 174.15 100.5) (layer Edge.Cuts) (width 0.2))
 (gr_line (start 175.15 117.15) (end 175.15 118.8) (layer Edge.Cuts) (width 0.2))
 (gr_circle (center 125.77 115.865) (end 127.29 115.865) (layer Edge.Cuts) (width 0.2))
 (gr_circle (center 139.17929 116.15) (end 141.92929 116.15) (layer Edge.Cuts) (width 0.2))
 (gr_circle (center 125.15 110.15) (end 126.05 110.15) (layer Edge.Cuts) (width 0.2))
 (gr_circle (center 132.12 110.785) (end 132.350001 110.785) (layer Edge.Cuts) (width 0.2))
 (gr_line (start 120.15 118.8) (end 120.15 101.5) (layer Edge.Cuts) (width 0.2))
 (gr_circle (center 132.12 108.245) (end 132.350001 108.245) (layer Edge.Cuts) (width 0.2))
 (gr_arc (start 174.15 118.8) (end 174.15 119.8) (angle -90) (layer Edge.Cuts) (width 0.2))
 (gr_circle (center 134.66 106.975) (end 134.89 106.975) (layer Edge.Cuts) (width 0.2))
 (gr_circle (center 134.66 109.515) (end 134.89 109.515) (layer Edge.Cuts) (width 0.2))
 (gr_circle (center 132.12 113.325) (end 132.35 113.325) (layer Edge.Cuts) (width 0.2))
 (gr_arc (start 173.85 114.15) (end 173.85 111.15) (angle -180) (layer Edge.Cuts) (width 0.2))
 (gr_line (start 175.15 101.5) (end 175.15 111.15) (layer Edge.Cuts) (width 0.2))
 (gr_circle (center 125.77 104.435) (end 127.29 104.435) (layer Edge.Cuts) (width 0.2))
 (gr_arc (start 121.15 101.5) (end 121.15 100.5) (angle -90) (layer Edge.Cuts) (width 0.2))
 (segment (start 162.68 113.3) (end 162.77 113.3) (width 0.25) (layer F.Cu) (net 2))
 (segment (start 163.025 113.555) (end 164.59 113.555) (width 0.25) (layer F.Cu) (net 2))
 (segment (start 162.77 113.3) (end 163.025 113.555) (width 0.25) (layer F.Cu) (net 2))
 (segment (start 162.255 114.81) (end 162.255 114.775) (width 0.25) (layer F.Cu) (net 2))
 (segment (start 161.63 114.15) (end 161.63 112.8) (width 0.25) (layer F.Cu) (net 2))
 (segment (start 162.255 114.775) (end 161.63 114.15) (width 0.25) (layer F.Cu) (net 2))
 (segment (start 162.13 113.3) (end 161.63 112.8) (width 0.25) (layer F.Cu) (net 2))
 (segment (start 162.68 113.3) (end 162.13 113.3) (width 0.25) (layer F.Cu) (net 2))
 (segment (start 162.23 110.82) (end 162.17 110.82) (width 0.25) (layer F.Cu) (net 2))
 (segment (start 161.63 111.36) (end 161.63 112.8) (width 0.25) (layer F.Cu) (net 2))
 (segment (start 162.17 110.82) (end 161.63 111.36) (width 0.25) (layer F.Cu) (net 2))
 (segment (start 160.68 112.2) (end 160.58 112.3) (width 0.25) (layer F.Cu) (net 15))
 (segment (start 160.68 110.82) (end 160.68 112.2) (width 0.25) (layer F.Cu) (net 15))
 (segment (start 162.68 112.3) (end 162.96 112.3) (width 0.25) (layer F.Cu) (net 4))
 (segment (start 163.255 112.005) (end 164.59 112.005) (width 0.25) (layer F.Cu) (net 4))
 (segment (start 162.96 112.3) (end 163.255 112.005) (width 0.25) (layer F.Cu) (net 4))
 (via (at 163.72 112.8) (size 0.6) (drill 0.3) (layers F.Cu B.Cu) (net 72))
 (segment (start 163.72 112.8) (end 162.68 112.8) (width 0.25) (layer F.Cu) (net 72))
 (segment (start 160.58 114.785) (end 160.605 114.81) (width 0.25) (layer F.Cu) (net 70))
 (segment (start 160.58 113.3) (end 160.58 114.785) (width 0.25) (layer F.Cu) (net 70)))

